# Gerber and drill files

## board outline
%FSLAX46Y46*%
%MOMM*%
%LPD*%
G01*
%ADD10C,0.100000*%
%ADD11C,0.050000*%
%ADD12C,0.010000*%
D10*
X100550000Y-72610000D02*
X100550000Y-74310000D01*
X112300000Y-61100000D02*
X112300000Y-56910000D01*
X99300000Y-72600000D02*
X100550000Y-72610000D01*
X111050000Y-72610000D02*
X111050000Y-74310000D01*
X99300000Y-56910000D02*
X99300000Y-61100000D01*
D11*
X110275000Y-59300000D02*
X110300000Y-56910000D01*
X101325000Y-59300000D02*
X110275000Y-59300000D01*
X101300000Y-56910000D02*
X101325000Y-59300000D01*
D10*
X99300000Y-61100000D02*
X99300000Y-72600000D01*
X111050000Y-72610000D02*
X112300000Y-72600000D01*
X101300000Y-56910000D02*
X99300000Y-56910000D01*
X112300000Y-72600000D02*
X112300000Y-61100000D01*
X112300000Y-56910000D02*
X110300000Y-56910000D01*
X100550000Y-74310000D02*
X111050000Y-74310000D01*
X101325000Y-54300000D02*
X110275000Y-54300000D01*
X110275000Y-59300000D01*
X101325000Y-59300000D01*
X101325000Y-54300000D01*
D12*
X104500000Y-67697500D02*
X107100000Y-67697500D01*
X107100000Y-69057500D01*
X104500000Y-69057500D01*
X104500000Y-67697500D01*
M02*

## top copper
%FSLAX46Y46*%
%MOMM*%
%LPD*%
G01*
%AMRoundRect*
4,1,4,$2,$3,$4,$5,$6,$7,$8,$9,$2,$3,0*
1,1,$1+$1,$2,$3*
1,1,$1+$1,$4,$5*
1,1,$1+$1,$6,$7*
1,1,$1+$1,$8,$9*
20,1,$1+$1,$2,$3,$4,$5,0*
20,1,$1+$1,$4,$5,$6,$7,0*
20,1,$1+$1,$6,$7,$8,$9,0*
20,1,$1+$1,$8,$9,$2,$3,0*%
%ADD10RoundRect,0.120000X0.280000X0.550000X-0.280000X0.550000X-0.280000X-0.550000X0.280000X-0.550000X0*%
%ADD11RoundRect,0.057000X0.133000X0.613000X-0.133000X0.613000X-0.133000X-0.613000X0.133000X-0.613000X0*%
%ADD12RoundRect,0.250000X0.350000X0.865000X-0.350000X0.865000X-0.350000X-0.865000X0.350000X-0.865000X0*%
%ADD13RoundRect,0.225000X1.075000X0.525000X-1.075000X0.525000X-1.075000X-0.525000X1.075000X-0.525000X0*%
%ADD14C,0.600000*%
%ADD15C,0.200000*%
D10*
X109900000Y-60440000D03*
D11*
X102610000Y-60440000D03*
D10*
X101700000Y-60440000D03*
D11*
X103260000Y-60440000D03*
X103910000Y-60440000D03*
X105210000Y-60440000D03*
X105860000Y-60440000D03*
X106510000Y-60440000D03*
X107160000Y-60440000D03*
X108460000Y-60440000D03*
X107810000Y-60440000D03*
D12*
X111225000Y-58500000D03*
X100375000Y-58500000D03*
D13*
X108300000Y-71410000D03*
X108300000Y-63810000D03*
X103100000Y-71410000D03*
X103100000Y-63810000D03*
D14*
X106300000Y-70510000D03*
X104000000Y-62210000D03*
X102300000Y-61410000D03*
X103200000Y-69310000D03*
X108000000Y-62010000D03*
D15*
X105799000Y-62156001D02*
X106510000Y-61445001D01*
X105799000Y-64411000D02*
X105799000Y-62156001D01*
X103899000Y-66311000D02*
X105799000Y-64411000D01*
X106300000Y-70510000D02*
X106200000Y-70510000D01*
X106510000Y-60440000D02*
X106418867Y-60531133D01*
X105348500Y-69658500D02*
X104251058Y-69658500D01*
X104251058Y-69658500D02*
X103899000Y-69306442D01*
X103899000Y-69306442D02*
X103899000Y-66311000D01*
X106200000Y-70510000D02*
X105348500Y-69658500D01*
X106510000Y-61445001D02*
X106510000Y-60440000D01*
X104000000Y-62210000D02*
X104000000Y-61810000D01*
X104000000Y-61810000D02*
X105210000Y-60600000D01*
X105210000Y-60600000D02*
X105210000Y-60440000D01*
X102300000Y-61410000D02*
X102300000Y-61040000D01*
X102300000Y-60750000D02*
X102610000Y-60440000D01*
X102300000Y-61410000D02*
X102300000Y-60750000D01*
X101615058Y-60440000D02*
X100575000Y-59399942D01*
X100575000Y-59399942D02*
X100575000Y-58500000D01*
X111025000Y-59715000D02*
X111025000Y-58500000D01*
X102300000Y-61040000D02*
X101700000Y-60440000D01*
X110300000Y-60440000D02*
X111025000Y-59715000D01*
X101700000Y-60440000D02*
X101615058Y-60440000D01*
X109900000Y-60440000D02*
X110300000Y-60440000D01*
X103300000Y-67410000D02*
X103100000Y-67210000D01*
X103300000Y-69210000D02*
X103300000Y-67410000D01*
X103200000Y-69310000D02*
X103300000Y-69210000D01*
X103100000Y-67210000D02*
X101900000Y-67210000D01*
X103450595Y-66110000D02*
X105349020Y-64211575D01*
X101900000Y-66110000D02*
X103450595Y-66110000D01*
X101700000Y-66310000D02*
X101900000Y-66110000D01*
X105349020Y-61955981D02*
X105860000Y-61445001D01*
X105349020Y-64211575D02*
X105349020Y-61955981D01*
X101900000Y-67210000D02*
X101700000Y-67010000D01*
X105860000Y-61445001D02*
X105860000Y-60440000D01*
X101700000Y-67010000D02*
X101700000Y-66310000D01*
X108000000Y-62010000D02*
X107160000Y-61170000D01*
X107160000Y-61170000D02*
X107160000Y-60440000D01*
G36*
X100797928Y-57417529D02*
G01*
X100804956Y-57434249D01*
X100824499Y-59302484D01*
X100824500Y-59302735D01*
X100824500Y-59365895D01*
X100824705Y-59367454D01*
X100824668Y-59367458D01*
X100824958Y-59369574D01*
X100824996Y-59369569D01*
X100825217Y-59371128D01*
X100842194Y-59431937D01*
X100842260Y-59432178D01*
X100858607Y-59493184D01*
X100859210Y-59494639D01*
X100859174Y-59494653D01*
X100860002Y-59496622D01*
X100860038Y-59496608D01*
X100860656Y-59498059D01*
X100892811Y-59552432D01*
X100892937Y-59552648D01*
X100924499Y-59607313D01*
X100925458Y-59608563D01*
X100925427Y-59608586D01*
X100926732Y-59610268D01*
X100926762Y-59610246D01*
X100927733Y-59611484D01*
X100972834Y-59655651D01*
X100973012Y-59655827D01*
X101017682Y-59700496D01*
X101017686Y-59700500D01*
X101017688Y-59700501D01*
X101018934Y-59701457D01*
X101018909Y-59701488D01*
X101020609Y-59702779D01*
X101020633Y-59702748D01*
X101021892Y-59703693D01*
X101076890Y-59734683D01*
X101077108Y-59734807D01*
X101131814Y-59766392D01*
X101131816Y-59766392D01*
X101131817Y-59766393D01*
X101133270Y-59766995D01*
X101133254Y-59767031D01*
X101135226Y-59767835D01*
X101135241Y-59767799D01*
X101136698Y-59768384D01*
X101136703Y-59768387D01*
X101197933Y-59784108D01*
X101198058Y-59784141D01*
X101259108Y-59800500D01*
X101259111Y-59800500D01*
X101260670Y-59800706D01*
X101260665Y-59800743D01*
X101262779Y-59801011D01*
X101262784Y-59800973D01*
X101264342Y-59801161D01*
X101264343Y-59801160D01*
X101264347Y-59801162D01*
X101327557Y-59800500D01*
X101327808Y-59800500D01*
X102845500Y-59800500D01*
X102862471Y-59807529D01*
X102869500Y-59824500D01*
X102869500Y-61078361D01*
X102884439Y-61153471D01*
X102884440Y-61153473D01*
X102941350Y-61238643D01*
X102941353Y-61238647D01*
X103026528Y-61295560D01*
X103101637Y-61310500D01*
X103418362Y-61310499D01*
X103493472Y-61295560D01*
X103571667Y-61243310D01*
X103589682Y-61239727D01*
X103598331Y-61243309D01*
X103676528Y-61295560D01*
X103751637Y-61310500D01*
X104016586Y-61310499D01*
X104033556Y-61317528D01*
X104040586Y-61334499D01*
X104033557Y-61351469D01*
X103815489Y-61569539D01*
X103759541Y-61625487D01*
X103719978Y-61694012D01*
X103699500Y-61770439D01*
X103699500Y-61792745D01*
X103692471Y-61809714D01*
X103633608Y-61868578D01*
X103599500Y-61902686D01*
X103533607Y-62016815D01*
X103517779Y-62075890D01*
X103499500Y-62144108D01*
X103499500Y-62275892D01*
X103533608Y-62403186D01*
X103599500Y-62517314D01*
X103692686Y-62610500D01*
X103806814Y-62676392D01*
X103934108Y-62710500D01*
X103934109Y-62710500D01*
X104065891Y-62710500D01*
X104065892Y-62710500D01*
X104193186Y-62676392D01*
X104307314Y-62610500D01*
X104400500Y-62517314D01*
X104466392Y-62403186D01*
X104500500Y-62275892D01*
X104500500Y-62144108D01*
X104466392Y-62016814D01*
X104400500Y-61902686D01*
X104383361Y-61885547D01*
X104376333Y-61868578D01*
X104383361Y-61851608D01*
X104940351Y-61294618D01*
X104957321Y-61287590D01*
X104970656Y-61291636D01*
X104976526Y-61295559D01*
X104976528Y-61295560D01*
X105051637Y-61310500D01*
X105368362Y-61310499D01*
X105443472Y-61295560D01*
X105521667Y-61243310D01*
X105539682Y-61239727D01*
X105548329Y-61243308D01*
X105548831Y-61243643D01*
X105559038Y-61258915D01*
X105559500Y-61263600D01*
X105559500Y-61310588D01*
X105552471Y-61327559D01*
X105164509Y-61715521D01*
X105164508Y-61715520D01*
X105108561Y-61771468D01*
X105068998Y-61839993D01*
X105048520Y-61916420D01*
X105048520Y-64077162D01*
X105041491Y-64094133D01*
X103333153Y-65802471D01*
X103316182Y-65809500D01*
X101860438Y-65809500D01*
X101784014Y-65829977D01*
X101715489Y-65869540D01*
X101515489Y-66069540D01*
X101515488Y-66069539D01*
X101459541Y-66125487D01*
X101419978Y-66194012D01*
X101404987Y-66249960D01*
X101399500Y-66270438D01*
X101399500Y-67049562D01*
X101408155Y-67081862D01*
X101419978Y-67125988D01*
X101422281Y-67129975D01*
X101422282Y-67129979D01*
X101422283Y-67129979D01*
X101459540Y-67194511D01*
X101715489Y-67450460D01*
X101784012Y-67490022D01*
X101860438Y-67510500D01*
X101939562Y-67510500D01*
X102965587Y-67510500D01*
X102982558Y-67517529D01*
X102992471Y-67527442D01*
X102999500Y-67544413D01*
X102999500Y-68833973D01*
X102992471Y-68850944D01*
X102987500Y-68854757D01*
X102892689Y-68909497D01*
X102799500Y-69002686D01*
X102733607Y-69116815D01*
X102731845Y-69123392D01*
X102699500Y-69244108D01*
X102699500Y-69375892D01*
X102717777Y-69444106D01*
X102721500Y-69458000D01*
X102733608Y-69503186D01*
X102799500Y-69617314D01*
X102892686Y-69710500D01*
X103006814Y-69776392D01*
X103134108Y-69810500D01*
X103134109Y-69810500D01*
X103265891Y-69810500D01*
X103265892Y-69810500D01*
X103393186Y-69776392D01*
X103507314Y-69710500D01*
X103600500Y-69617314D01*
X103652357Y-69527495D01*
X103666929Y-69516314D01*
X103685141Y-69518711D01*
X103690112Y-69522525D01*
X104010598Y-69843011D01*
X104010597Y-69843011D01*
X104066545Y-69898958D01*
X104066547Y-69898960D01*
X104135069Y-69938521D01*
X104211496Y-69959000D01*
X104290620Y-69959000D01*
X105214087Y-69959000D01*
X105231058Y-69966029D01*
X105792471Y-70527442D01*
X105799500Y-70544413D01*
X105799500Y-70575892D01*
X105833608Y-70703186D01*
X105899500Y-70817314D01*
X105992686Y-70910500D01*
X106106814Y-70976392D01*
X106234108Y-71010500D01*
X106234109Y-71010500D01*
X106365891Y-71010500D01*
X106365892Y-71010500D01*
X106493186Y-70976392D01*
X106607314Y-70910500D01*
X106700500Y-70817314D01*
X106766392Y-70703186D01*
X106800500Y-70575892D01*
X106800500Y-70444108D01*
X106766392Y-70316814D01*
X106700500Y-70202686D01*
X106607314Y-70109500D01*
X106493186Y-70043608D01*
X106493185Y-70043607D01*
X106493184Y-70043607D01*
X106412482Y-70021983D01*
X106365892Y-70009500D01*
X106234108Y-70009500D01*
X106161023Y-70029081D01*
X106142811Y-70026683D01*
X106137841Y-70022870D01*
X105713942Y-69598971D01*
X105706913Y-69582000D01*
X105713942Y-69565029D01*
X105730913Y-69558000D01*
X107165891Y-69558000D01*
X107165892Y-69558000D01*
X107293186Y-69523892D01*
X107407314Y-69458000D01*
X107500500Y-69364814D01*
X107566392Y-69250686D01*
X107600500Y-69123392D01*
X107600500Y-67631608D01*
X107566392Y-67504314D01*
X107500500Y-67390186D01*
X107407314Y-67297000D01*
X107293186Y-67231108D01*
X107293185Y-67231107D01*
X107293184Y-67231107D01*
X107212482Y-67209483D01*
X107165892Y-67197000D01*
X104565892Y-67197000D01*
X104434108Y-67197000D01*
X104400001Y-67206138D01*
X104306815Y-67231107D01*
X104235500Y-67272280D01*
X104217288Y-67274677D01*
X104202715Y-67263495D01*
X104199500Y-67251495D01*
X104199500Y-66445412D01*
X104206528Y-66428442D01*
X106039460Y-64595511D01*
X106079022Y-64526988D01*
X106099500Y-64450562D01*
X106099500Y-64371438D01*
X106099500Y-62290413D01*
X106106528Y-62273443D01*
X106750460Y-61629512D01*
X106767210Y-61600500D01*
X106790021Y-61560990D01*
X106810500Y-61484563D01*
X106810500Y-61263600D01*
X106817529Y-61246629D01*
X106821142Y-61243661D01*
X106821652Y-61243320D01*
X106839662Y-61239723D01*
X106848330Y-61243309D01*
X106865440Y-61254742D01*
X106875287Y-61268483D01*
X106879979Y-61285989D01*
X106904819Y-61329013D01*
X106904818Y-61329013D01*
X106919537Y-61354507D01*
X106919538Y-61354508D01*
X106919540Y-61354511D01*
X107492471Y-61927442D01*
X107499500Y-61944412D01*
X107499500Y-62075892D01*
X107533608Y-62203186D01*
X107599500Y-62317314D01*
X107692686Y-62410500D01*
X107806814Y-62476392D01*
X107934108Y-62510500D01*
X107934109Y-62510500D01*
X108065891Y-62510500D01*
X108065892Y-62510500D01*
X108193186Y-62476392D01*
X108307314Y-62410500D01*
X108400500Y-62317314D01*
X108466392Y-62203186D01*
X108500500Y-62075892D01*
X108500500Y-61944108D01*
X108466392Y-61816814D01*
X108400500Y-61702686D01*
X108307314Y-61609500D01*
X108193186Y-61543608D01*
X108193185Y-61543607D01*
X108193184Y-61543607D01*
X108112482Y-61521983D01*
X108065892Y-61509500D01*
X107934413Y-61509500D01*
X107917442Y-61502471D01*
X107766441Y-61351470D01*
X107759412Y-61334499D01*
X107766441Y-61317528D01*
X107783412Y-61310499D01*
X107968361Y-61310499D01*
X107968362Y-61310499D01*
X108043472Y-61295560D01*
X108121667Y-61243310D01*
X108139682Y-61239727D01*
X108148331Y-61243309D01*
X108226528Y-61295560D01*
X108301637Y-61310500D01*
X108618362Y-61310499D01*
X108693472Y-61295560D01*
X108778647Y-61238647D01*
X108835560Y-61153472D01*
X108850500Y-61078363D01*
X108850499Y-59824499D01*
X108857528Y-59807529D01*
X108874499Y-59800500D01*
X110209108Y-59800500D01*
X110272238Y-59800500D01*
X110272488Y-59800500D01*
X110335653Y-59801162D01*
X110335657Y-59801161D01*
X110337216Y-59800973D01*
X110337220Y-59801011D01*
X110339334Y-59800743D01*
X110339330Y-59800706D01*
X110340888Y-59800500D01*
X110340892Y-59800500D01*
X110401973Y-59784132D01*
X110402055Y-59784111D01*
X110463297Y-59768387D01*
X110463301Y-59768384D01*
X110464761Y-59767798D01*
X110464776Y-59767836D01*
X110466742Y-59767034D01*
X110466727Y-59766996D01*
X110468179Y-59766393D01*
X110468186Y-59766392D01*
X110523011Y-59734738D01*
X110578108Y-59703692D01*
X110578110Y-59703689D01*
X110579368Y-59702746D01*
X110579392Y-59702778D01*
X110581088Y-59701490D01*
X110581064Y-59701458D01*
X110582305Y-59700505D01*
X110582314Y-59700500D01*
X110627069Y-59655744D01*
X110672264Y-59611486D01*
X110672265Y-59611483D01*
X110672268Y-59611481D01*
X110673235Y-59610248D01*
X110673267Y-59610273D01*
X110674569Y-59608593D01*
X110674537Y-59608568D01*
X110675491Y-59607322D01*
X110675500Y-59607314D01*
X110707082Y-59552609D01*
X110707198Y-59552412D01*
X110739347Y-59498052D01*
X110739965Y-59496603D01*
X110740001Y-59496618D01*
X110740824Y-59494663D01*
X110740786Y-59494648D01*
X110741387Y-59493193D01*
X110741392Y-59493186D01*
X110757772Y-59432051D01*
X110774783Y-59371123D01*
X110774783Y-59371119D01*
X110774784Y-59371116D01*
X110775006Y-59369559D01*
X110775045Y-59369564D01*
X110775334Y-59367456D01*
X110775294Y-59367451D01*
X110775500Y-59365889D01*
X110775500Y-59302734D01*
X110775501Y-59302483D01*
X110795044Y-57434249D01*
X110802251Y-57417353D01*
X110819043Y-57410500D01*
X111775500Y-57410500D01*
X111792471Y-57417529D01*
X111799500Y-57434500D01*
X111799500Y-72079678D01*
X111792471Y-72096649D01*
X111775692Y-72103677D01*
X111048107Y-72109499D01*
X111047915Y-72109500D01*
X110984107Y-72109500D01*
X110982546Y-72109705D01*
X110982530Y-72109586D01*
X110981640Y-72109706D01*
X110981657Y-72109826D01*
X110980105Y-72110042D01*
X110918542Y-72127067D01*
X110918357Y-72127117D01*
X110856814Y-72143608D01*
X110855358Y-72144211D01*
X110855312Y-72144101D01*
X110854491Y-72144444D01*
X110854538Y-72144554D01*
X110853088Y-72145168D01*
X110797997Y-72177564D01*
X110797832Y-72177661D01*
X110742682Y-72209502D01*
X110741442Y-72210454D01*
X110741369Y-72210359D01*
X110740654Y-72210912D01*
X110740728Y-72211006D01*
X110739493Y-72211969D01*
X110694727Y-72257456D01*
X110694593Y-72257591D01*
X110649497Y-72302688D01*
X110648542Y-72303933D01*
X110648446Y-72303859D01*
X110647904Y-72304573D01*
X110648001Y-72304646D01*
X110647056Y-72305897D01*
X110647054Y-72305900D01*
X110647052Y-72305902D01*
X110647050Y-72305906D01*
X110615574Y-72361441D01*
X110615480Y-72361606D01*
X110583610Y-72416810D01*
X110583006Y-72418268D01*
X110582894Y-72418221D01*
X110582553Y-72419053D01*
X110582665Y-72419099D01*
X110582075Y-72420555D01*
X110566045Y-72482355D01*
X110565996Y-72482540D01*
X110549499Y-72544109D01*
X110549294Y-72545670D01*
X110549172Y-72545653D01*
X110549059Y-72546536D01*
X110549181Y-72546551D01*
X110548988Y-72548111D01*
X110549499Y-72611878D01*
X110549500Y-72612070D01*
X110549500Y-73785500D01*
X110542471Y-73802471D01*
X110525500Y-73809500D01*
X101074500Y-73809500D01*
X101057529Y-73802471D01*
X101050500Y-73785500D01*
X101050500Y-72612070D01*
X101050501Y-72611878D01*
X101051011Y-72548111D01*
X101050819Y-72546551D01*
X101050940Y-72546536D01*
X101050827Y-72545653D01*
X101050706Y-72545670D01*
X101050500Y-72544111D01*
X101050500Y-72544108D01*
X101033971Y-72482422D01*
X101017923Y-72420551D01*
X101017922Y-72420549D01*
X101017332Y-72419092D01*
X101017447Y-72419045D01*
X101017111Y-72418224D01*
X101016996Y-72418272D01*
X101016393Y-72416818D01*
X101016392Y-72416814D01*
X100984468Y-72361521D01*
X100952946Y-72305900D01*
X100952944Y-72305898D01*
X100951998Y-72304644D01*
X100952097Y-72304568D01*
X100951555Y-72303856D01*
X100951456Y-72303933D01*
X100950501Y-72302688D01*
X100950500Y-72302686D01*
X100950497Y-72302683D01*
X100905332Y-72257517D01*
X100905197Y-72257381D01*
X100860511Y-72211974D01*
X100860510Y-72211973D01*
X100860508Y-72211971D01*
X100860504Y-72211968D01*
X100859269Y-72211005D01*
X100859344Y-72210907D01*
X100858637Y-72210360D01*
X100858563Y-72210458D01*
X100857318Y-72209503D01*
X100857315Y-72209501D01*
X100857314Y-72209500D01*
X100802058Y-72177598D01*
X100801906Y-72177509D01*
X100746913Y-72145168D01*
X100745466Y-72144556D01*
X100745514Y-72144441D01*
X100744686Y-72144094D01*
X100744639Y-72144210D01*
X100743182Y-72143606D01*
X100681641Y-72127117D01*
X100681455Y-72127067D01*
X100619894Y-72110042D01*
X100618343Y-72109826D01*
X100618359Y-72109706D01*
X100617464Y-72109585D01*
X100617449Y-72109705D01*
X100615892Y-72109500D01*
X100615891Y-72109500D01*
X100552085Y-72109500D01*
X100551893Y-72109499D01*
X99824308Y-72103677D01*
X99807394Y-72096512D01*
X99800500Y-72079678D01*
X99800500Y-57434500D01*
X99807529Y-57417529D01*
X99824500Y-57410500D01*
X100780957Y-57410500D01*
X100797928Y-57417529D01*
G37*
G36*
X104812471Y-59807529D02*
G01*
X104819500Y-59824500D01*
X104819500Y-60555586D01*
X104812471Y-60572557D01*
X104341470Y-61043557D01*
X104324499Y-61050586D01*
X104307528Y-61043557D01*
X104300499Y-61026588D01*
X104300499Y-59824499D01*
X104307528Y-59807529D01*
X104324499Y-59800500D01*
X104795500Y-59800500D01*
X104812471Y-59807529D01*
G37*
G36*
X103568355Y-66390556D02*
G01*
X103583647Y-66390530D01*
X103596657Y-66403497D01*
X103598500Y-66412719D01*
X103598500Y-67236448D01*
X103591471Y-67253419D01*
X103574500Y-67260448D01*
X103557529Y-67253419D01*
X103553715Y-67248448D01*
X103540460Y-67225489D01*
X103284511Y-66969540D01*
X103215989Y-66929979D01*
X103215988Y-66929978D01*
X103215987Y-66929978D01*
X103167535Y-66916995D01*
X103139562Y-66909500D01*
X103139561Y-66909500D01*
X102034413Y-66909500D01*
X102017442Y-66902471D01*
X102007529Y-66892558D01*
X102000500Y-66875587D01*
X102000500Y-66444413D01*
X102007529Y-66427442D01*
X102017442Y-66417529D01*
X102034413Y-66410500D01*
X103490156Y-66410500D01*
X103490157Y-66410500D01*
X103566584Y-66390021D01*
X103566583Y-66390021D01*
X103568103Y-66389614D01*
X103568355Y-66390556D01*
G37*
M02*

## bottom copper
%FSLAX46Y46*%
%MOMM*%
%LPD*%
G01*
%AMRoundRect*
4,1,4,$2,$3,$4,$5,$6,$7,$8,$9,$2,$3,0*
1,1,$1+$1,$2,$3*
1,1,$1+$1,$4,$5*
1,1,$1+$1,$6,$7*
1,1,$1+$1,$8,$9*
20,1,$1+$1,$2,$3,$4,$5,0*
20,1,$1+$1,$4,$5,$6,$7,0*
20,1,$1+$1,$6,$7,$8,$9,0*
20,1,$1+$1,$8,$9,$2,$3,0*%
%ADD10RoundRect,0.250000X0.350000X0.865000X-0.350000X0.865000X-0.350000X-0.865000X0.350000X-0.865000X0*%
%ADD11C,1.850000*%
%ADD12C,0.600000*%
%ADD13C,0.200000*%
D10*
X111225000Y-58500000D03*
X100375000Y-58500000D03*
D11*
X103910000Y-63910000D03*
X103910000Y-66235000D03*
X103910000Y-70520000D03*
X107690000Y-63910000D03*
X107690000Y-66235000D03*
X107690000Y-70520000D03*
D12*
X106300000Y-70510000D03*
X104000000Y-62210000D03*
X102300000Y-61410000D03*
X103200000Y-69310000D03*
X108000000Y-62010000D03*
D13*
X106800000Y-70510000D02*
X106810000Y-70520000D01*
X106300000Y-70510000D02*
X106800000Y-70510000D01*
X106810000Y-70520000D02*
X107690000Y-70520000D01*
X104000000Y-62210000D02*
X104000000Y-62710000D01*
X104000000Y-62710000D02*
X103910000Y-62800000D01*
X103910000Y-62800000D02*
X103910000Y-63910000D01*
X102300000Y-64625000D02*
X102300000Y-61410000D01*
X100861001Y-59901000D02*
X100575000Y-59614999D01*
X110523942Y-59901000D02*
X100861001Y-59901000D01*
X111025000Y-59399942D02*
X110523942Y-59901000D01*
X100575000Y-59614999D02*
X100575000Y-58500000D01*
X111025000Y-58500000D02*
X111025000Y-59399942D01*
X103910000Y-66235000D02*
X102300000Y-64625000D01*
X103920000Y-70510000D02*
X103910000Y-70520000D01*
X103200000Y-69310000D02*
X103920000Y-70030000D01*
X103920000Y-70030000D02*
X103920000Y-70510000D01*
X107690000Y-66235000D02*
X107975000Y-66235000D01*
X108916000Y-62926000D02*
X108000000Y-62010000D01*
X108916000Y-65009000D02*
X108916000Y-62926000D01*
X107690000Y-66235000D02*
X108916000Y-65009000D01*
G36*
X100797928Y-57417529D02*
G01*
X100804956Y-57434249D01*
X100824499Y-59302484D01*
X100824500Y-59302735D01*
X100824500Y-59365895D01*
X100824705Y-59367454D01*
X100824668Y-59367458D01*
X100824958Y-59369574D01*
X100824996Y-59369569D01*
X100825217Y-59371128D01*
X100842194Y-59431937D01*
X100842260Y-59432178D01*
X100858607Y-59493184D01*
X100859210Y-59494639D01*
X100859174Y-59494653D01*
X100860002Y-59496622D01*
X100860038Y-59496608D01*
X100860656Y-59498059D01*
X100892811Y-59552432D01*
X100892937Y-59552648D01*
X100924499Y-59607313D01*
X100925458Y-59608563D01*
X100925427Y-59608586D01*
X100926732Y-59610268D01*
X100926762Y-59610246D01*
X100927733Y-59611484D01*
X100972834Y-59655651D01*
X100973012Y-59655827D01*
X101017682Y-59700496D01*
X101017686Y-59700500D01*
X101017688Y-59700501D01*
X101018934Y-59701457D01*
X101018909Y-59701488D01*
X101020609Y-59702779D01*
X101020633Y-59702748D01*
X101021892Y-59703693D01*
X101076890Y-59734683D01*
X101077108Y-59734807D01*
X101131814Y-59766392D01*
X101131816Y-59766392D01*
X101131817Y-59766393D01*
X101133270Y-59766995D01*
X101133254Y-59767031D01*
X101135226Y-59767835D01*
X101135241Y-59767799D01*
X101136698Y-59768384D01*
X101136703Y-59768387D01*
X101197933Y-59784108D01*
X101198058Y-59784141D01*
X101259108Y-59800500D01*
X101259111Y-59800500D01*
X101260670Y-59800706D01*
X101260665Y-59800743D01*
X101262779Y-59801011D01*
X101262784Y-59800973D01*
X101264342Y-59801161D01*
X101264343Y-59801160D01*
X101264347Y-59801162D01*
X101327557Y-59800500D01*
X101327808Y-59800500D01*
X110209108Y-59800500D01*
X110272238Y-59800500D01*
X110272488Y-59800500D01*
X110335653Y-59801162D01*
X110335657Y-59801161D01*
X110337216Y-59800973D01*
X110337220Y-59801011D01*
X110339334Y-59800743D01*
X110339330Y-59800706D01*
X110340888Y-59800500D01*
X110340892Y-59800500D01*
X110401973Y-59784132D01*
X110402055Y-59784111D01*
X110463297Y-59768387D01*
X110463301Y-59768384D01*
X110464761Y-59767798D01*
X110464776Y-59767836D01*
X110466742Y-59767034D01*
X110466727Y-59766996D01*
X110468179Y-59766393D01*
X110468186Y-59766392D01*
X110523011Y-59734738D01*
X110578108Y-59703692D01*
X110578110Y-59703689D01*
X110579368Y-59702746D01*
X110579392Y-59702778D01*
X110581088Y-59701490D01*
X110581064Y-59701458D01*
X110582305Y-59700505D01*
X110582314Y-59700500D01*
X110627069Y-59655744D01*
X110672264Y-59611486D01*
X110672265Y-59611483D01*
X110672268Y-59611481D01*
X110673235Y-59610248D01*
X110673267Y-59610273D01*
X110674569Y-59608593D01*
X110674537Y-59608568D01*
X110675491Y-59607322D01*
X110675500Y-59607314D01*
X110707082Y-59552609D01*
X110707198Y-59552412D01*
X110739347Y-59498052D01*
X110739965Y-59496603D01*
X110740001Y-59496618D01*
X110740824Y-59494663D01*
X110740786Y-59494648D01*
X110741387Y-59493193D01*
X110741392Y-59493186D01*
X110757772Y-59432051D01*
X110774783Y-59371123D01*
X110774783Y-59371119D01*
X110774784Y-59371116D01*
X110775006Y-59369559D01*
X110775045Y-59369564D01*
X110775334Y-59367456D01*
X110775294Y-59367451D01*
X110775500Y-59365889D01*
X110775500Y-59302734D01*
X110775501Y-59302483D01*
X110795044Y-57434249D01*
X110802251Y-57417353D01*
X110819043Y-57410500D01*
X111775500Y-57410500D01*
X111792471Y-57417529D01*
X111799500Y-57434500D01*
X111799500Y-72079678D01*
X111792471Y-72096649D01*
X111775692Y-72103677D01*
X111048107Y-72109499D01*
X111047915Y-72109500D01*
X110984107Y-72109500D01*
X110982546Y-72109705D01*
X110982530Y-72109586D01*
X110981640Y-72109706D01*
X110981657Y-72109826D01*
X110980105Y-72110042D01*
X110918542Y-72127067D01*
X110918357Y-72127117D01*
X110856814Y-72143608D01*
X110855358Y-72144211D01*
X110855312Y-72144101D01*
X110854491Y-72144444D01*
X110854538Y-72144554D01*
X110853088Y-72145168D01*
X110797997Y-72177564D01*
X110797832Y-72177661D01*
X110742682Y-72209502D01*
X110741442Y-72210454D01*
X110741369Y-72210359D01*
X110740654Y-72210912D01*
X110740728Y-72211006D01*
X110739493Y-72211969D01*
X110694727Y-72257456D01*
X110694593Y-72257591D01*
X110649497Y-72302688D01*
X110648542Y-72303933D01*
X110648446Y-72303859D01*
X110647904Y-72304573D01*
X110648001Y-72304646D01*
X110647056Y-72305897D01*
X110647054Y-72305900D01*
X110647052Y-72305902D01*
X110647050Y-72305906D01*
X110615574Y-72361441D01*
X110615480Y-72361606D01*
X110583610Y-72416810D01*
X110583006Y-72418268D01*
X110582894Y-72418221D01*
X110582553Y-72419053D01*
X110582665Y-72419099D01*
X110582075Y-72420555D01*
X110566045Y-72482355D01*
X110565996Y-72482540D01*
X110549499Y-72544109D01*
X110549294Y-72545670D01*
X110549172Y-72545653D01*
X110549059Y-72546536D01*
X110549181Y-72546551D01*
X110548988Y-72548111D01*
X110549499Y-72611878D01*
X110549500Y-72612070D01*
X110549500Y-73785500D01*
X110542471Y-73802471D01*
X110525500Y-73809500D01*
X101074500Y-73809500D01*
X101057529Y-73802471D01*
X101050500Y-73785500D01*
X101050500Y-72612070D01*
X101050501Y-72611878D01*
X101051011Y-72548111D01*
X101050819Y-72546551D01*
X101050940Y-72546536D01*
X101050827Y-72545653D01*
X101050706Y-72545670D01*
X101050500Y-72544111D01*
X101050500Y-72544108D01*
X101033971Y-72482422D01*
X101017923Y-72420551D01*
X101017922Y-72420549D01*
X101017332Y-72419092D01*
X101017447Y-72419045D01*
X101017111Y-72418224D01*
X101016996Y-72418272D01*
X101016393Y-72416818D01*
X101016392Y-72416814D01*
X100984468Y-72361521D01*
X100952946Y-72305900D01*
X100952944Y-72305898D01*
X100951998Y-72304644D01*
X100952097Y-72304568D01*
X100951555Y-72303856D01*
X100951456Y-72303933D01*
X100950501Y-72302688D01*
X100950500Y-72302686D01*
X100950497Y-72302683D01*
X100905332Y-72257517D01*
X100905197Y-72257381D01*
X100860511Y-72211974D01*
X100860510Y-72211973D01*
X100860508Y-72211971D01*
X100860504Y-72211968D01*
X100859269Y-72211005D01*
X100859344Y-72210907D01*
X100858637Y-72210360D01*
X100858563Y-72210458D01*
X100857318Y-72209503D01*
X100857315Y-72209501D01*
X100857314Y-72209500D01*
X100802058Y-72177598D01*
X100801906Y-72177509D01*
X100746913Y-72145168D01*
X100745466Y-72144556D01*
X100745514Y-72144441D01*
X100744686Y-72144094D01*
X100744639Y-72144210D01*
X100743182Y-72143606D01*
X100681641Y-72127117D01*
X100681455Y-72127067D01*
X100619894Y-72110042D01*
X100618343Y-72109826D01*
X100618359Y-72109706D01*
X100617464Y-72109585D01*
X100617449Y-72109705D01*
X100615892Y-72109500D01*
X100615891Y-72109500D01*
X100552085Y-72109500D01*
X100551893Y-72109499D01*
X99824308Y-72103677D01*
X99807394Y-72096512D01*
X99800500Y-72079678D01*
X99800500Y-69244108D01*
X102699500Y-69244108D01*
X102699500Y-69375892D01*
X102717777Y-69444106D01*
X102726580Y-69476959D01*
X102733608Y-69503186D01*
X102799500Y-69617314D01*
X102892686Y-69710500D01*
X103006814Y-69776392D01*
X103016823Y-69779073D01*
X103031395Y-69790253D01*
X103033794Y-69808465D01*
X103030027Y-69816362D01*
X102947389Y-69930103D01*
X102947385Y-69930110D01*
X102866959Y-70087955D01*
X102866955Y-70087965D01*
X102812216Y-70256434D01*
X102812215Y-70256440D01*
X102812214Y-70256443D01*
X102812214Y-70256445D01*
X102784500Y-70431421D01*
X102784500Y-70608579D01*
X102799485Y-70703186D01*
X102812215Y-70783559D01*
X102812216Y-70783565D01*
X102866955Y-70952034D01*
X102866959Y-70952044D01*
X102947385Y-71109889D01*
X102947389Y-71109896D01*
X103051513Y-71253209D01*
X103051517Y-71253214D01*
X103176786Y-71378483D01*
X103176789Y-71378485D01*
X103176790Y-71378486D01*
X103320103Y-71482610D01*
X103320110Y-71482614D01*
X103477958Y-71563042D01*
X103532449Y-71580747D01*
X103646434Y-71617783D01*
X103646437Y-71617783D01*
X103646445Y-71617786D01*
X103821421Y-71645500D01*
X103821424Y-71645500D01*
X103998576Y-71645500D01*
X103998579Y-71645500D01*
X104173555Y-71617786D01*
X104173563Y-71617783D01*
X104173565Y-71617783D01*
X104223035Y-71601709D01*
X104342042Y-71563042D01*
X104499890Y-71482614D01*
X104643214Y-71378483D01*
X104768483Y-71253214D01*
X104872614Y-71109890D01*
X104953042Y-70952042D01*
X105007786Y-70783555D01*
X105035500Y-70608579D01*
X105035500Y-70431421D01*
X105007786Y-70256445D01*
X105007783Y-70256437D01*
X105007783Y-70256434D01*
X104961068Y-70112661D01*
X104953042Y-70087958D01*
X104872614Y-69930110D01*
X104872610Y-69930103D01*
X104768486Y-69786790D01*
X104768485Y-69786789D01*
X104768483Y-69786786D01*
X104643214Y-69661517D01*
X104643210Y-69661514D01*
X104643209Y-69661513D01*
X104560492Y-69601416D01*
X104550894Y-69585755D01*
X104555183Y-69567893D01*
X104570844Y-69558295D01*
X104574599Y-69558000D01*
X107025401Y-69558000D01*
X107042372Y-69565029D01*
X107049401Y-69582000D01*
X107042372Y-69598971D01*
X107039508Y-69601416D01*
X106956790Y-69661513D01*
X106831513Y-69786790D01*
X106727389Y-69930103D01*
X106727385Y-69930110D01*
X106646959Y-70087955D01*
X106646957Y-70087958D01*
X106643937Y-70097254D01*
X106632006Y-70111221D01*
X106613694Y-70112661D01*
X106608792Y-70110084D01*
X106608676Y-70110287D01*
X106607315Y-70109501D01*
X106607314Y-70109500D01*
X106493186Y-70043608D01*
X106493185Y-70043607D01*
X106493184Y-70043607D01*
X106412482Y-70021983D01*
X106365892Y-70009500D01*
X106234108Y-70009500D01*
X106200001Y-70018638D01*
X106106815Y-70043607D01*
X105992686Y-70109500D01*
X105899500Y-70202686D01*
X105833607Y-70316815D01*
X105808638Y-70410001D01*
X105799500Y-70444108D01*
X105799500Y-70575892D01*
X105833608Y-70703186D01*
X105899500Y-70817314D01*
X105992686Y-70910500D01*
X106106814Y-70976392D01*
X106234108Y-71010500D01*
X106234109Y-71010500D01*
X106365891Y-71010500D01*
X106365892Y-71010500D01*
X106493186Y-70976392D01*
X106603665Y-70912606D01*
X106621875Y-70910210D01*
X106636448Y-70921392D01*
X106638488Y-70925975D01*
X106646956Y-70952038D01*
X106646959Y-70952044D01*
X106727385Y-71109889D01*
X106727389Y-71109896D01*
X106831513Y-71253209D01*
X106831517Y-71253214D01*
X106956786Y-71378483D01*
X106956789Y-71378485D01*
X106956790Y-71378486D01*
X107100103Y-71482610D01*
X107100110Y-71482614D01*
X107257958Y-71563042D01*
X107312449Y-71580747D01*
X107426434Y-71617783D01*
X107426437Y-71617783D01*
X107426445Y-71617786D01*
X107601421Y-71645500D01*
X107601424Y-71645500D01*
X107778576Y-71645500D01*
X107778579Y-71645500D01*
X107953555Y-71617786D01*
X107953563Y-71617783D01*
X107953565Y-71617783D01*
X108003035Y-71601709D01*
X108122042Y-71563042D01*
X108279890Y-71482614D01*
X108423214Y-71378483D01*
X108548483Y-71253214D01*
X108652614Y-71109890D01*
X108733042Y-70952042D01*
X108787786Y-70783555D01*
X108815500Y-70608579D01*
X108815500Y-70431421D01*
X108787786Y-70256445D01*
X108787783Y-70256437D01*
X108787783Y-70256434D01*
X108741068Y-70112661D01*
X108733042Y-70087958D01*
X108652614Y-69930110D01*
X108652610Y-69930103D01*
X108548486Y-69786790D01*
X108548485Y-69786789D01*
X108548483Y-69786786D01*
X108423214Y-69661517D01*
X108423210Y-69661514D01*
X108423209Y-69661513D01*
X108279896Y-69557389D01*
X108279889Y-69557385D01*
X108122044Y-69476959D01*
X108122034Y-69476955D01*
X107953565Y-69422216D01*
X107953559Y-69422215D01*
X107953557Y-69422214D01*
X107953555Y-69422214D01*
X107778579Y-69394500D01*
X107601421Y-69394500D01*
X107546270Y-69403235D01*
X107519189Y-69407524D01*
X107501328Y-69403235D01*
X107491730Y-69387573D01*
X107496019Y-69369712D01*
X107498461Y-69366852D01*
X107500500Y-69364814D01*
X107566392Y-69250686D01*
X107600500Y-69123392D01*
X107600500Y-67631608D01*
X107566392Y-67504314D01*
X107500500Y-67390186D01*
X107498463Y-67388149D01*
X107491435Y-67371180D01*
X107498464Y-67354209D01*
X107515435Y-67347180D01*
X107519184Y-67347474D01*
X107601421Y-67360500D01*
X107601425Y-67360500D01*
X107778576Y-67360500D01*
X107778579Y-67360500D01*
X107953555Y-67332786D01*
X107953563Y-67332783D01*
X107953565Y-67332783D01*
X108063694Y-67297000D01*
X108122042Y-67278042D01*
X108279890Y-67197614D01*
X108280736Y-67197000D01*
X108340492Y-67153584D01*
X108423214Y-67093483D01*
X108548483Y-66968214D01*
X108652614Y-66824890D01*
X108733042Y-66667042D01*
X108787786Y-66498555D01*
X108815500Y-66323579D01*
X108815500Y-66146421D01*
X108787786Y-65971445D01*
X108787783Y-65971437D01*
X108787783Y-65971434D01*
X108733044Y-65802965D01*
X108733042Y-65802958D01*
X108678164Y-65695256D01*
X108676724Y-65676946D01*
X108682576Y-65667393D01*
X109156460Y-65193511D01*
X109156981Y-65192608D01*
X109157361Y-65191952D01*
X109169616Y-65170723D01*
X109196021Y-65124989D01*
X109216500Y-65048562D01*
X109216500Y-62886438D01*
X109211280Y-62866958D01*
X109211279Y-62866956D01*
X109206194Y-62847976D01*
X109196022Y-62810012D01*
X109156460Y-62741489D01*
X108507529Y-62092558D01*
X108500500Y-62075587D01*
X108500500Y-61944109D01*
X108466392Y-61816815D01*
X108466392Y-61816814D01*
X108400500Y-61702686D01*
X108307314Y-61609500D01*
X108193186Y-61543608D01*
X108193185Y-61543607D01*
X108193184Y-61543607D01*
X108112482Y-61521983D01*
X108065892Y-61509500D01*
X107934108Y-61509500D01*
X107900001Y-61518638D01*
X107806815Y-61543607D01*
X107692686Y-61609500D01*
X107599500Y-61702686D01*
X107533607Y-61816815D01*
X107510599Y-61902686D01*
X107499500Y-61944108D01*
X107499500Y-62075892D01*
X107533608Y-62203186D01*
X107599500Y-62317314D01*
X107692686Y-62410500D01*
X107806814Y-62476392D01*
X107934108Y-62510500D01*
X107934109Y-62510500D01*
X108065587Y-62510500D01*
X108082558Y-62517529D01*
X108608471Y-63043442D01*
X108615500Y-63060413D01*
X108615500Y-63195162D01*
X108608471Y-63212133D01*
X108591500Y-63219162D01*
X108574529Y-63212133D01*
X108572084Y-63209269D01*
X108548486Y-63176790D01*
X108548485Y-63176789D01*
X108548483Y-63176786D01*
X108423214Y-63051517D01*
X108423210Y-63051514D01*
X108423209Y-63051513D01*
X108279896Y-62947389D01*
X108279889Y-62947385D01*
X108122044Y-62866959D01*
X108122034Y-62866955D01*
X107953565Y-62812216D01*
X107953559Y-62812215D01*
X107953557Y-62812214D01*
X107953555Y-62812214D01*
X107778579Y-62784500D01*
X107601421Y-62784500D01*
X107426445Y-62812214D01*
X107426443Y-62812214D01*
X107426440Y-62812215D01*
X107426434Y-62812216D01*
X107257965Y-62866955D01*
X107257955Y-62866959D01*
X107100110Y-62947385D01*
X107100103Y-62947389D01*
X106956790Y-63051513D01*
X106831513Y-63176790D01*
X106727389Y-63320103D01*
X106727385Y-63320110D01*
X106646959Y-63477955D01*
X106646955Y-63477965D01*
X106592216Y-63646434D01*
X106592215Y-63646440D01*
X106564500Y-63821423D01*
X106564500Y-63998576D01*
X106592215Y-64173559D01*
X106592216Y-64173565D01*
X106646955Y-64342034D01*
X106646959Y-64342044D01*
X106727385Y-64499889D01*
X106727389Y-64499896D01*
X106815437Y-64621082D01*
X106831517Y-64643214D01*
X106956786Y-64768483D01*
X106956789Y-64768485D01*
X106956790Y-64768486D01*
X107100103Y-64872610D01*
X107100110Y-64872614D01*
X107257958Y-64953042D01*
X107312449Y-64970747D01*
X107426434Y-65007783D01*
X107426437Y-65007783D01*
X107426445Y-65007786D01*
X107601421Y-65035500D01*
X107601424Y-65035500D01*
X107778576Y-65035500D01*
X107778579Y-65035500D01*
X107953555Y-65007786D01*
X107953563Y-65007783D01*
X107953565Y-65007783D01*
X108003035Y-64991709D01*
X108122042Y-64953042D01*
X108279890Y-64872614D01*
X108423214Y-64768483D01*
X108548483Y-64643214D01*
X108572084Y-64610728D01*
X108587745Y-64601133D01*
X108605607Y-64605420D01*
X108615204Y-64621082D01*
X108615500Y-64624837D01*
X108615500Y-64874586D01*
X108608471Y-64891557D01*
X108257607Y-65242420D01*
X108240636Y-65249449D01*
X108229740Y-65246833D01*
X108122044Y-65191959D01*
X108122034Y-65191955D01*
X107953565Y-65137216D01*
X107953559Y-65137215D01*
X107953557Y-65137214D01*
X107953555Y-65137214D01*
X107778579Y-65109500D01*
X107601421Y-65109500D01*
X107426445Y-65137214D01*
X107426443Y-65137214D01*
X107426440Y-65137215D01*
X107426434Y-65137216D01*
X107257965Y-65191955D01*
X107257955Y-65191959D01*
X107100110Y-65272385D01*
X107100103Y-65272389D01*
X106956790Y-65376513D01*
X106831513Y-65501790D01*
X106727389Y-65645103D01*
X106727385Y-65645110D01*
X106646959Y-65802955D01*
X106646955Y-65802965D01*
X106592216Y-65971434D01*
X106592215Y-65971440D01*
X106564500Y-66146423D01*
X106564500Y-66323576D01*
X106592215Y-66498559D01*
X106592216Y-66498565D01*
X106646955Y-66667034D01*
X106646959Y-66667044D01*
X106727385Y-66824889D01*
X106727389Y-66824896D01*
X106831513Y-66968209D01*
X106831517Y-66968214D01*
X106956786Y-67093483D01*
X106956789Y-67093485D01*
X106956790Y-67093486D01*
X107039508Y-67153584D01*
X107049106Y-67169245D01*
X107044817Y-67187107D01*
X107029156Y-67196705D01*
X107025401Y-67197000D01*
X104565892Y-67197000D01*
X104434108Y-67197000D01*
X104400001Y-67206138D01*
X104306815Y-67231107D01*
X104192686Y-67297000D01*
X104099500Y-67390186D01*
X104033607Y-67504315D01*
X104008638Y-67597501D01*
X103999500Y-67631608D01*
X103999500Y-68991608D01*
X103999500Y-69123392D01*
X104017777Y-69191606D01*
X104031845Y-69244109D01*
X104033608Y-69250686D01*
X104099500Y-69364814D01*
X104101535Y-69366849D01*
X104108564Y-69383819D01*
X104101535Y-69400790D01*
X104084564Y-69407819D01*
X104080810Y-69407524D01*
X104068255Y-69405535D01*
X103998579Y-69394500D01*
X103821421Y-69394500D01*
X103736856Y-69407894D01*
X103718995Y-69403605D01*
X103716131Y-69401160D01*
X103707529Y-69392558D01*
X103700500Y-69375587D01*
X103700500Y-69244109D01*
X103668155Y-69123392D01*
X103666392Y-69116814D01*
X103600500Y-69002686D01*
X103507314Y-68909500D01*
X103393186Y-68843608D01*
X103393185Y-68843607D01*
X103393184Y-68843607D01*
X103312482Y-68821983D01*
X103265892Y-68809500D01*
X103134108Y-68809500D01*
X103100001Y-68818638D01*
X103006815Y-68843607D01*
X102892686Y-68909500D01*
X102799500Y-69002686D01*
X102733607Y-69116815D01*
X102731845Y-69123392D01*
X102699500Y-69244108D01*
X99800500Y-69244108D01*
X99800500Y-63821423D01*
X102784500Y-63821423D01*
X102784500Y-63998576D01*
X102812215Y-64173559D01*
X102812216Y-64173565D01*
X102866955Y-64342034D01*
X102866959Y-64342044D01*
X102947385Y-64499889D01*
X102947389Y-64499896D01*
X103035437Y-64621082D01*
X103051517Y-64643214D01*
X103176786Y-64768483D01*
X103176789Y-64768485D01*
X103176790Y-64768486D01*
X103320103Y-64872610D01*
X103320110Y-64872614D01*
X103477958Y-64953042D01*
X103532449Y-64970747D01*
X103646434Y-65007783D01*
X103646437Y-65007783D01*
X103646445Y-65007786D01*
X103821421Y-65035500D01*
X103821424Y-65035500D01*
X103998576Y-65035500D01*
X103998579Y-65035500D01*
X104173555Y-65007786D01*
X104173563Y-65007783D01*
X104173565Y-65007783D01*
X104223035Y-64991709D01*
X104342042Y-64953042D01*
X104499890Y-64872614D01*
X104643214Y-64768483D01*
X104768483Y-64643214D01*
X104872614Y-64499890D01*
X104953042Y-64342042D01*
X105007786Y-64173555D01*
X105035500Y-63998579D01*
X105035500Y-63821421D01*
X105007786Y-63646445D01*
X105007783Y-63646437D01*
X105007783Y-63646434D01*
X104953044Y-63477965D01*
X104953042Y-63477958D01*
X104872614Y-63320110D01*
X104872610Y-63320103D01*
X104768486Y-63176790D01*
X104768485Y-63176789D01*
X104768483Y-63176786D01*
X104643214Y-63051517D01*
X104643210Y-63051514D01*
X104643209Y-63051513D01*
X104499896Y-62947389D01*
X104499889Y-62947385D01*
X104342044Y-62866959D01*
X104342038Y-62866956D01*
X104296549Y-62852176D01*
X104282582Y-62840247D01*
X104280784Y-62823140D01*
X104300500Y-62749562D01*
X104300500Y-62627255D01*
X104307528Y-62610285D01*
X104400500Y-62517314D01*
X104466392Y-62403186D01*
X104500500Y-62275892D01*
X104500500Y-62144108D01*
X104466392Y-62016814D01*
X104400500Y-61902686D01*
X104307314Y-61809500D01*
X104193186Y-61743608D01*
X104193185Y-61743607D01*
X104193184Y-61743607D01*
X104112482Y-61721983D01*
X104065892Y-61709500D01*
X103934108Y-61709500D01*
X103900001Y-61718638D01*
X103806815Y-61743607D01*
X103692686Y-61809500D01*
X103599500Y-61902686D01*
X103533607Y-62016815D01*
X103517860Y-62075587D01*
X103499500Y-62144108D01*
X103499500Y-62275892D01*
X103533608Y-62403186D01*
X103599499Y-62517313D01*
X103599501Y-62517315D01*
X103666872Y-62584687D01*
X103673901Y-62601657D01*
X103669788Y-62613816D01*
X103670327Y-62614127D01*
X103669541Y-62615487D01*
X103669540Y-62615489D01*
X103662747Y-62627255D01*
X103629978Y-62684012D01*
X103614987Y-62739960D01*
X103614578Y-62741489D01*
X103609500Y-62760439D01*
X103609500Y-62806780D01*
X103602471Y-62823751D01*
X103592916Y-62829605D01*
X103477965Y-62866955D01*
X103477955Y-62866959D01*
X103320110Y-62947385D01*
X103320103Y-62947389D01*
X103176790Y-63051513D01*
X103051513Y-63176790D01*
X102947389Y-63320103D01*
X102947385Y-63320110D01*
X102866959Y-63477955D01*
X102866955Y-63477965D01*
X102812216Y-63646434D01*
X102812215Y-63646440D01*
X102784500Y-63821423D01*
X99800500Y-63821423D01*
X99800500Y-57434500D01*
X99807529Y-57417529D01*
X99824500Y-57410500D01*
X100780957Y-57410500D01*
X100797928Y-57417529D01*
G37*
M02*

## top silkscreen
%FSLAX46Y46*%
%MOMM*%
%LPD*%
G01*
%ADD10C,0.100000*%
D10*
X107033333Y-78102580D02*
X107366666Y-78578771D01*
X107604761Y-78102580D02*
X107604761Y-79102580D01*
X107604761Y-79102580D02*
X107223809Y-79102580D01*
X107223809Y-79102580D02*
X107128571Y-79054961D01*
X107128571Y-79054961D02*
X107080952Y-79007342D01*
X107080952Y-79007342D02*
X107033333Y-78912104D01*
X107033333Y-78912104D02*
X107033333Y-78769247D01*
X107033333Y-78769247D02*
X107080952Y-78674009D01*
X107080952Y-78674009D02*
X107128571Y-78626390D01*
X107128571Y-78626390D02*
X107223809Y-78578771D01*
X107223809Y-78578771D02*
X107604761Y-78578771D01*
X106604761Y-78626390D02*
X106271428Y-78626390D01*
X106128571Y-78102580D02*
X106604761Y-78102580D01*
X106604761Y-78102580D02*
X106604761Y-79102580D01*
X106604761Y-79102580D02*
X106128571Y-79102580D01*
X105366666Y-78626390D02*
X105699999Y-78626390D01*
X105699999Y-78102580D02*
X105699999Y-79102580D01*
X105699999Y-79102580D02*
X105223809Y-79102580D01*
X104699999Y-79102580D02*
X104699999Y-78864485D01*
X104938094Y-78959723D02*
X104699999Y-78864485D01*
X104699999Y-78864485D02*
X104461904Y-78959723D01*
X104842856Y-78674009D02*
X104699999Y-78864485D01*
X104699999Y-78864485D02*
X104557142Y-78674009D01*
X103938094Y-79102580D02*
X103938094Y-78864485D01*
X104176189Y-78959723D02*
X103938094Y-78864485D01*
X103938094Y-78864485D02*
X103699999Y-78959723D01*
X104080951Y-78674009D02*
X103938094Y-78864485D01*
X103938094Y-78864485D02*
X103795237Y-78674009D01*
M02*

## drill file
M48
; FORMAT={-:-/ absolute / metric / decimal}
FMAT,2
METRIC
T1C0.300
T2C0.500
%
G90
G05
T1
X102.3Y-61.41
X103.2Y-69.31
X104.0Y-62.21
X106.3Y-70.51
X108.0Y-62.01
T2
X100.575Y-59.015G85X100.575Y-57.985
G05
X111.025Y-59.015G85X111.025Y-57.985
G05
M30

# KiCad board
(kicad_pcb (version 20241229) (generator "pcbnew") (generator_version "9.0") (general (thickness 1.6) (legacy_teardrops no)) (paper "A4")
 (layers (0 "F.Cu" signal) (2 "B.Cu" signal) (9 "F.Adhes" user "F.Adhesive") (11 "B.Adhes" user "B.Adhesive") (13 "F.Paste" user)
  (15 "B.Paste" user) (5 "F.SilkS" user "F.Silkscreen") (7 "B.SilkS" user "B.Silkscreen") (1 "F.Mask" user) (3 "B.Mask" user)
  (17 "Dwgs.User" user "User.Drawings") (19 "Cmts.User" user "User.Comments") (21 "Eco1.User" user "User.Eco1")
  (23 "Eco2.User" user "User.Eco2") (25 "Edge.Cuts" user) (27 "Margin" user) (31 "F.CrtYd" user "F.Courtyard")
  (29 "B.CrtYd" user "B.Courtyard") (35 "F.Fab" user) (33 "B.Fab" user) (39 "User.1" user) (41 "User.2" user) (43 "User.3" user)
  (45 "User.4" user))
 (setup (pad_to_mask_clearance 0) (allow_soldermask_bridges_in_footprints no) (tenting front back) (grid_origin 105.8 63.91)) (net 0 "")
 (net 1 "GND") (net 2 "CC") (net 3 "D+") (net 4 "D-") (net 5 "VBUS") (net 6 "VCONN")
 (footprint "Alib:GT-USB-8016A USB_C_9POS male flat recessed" (layer "F.Cu") (at 105.8 62 180)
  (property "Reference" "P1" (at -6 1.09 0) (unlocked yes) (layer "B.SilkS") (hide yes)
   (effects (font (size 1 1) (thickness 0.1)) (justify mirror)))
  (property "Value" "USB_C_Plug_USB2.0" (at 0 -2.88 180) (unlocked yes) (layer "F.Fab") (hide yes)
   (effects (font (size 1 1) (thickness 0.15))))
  (fp_rect (start -4.475 2.7) (end 4.475 7.7) (stroke (width 0.1) (type solid)) (fill no) (layer "Edge.Cuts"))
  (pad "A1" smd roundrect (at -4.1 1.56 180) (size 0.8 1.34) (layers "F.Cu" "F.Mask" "F.Paste") (roundrect_rratio 0.15) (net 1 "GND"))
  (pad "A1" smd roundrect (at 3.19 1.56 180) (size 0.38 1.34) (layers "F.Cu" "F.Mask" "F.Paste") (roundrect_rratio 0.15) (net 1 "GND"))
  (pad "A1" smd roundrect (at 4.1 1.56 180) (size 0.8 1.34) (layers "F.Cu" "F.Mask" "F.Paste") (roundrect_rratio 0.15) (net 1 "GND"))
  (pad "A2" smd roundrect (at 2.54 1.56 180) (size 0.38 1.34) (layers "F.Cu" "F.Mask" "F.Paste") (roundrect_rratio 0.15))
  (pad "A3" smd roundrect (at 1.89 1.56 180) (size 0.38 1.34) (layers "F.Cu" "F.Mask" "F.Paste") (roundrect_rratio 0.15))
  (pad "A5" smd roundrect (at 0.59 1.56 180) (size 0.38 1.34) (layers "F.Cu" "F.Mask" "F.Paste") (roundrect_rratio 0.15) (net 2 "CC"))
  (pad "A6" smd roundrect (at -0.06 1.56 180) (size 0.38 1.34) (layers "F.Cu" "F.Mask" "F.Paste") (roundrect_rratio 0.15) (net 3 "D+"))
  (pad "A7" smd roundrect (at -0.71 1.56 180) (size 0.38 1.34) (layers "F.Cu" "F.Mask" "F.Paste") (roundrect_rratio 0.15) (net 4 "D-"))
  (pad "A9" smd roundrect (at -1.36 1.56 180) (size 0.38 1.34) (layers "F.Cu" "F.Mask" "F.Paste") (roundrect_rratio 0.15) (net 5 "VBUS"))
  (pad "B10" smd roundrect (at -2.66 1.56 180) (size 0.38 1.34) (layers "F.Cu" "F.Mask" "F.Paste") (roundrect_rratio 0.15))
  (pad "B11" smd roundrect (at -2.01 1.56 180) (size 0.38 1.34) (layers "F.Cu" "F.Mask" "F.Paste") (roundrect_rratio 0.15))
  (pad "S1" thru_hole roundrect (at -5.225 3.5 180) (size 1.2 2.23) (drill oval 0.5 1.53 (offset -0.2 0)) (layers "*.Cu" "*.Mask")
   (remove_unused_layers no) (roundrect_rratio 0.2083333333) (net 1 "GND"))
  (pad "S1" thru_hole roundrect (at 5.225 3.5 180) (size 1.2 2.23) (drill oval 0.5 1.53 (offset 0.2 0)) (layers "*.Cu" "*.Mask")
   (remove_unused_layers no) (roundrect_rratio 0.2083333333) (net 1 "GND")))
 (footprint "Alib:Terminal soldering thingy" (layer "F.Cu") (at 105.7 78.06 180)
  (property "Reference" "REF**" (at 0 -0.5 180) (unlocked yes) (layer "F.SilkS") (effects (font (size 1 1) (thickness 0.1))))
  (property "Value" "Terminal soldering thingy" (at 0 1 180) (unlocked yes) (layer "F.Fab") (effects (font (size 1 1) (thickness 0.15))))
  (pad "1" smd roundrect (at -2.6 6.65 180) (size 2.6 1.5) (layers "F.Cu" "F.Mask" "F.Paste") (roundrect_rratio 0.15) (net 1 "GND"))
  (pad "1" smd roundrect (at -2.6 14.25 180) (size 2.6 1.5) (layers "F.Cu" "F.Mask" "F.Paste") (roundrect_rratio 0.15) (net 1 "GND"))
  (pad "1" smd roundrect (at 2.6 6.65 180) (size 2.6 1.5) (layers "F.Cu" "F.Mask" "F.Paste") (roundrect_rratio 0.15) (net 1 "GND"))
  (pad "1" smd roundrect (at 2.6 14.25 180) (size 2.6 1.5) (layers "F.Cu" "F.Mask" "F.Paste") (roundrect_rratio 0.15) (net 1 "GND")))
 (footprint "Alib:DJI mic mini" (layer "B.Cu") (at 105.8 63.91 180)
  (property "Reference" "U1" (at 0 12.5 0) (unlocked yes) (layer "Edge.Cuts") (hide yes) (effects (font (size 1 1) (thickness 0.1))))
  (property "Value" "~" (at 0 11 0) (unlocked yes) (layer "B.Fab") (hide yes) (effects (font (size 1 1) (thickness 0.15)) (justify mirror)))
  (fp_rect (start -1.3 -3.7875) (end 1.3 -5.1475) (stroke (width 0.01) (type solid)) (fill no) (layer "Edge.Cuts"))
  (pad "1" smd circle (at 1.89 0 180) (size 1.85 1.85) (layers "B.Cu" "B.Mask" "B.Paste") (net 2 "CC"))
  (pad "2" smd circle (at 1.89 -2.325 180) (size 1.85 1.85) (layers "B.Cu" "B.Mask" "B.Paste") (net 1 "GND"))
  (pad "3" smd circle (at 1.89 -6.61 180) (size 1.85 1.85) (layers "B.Cu" "B.Mask" "B.Paste") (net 3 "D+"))
  (pad "4" smd circle (at -1.89 0 180) (size 1.85 1.85) (layers "B.Cu" "B.Mask" "B.Paste") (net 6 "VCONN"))
  (pad "5" smd circle (at -1.89 -2.325 180) (size 1.85 1.85) (layers "B.Cu" "B.Mask" "B.Paste") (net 5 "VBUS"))
  (pad "6" smd circle (at -1.89 -6.61 180) (size 1.85 1.85) (layers "B.Cu" "B.Mask" "B.Paste") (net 4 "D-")))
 (gr_line (start 100.55 72.61) (end 100.55 74.31) (stroke (width 0.1) (type solid)) (layer "Edge.Cuts"))
 (gr_line (start 112.3 61.1) (end 112.3 56.91) (stroke (width 0.1) (type solid)) (layer "Edge.Cuts"))
 (gr_line (start 99.3 72.6) (end 100.55 72.61) (stroke (width 0.1) (type solid)) (layer "Edge.Cuts"))
 (gr_line (start 111.05 72.61) (end 111.05 74.31) (stroke (width 0.1) (type solid)) (layer "Edge.Cuts"))
 (gr_line (start 99.3 56.91) (end 99.3 61.1) (stroke (width 0.1) (type solid)) (layer "Edge.Cuts"))
 (gr_line (start 110.275 59.3) (end 110.3 56.91) (stroke (width 0.05) (type solid)) (layer "Edge.Cuts"))
 (gr_line (start 101.325 59.3) (end 110.275 59.3) (stroke (width 0.05) (type default)) (layer "Edge.Cuts"))
 (gr_line (start 101.3 56.91) (end 101.325 59.3) (stroke (width 0.05) (type default)) (layer "Edge.Cuts"))
 (gr_line (start 99.3 61.1) (end 99.3 72.6) (stroke (width 0.1) (type solid)) (layer "Edge.Cuts"))
 (gr_line (start 111.05 72.61) (end 112.3 72.6) (stroke (width 0.1) (type solid)) (layer "Edge.Cuts"))
 (gr_line (start 101.3 56.91) (end 99.3 56.91) (stroke (width 0.1) (type solid)) (layer "Edge.Cuts"))
 (gr_line (start 112.3 72.6) (end 112.3 61.1) (stroke (width 0.1) (type solid)) (layer "Edge.Cuts"))
 (gr_line (start 112.3 56.91) (end 110.3 56.91) (stroke (width 0.1) (type solid)) (layer "Edge.Cuts"))
 (gr_line (start 100.55 74.31) (end 111.05 74.31) (stroke (width 0.1) (type solid)) (layer "Edge.Cuts"))
 (segment (start 105.799 62.156001) (end 106.51 61.445001) (width 0.2) (layer "F.Cu") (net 4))
 (segment (start 105.799 64.411) (end 105.799 62.156001) (width 0.2) (layer "F.Cu") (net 4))
 (segment (start 103.899 66.311) (end 105.799 64.411) (width 0.2) (layer "F.Cu") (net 4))
 (segment (start 106.3 70.51) (end 106.2 70.51) (width 0.2) (layer "F.Cu") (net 4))
 (segment (start 106.51 60.44) (end 106.418867 60.531133) (width 0.2) (layer "F.Cu") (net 4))
 (segment (start 105.3485 69.6585) (end 104.251058 69.6585) (width 0.2) (layer "F.Cu") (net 4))
 (segment (start 104.251058 69.6585) (end 103.899 69.306442) (width 0.2) (layer "F.Cu") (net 4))
 (segment (start 103.899 69.306442) (end 103.899 66.311) (width 0.2) (layer "F.Cu") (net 4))
 (segment (start 106.2 70.51) (end 105.3485 69.6585) (width 0.2) (layer "F.Cu") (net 4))
 (segment (start 106.51 61.445001) (end 106.51 60.44) (width 0.2) (layer "F.Cu") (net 4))
 (via (at 106.3 70.51) (size 0.6) (drill 0.3) (layers "F.Cu" "B.Cu") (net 4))
 (segment (start 106.8 70.51) (end 106.81 70.52) (width 0.2) (layer "B.Cu") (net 4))
 (segment (start 106.3 70.51) (end 106.8 70.51) (width 0.2) (layer "B.Cu") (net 4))
 (segment (start 106.81 70.52) (end 107.69 70.52) (width 0.2) (layer "B.Cu") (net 4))
 (segment (start 104 62.21) (end 104 61.81) (width 0.2) (layer "F.Cu") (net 2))
 (segment (start 104 61.81) (end 105.21 60.6) (width 0.2) (layer "F.Cu") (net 2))
 (segment (start 105.21 60.6) (end 105.21 60.44) (width 0.2) (layer "F.Cu") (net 2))
 (via (at 104 62.21) (size 0.6) (drill 0.3) (layers "F.Cu" "B.Cu") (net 2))
 (segment (start 104 62.21) (end 104 62.71) (width 0.2) (layer "B.Cu") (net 2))
 (segment (start 104 62.71) (end 103.91 62.8) (width 0.2) (layer "B.Cu") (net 2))
 (segment (start 103.91 62.8) (end 103.91 63.91) (width 0.2) (layer "B.Cu") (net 2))
 (segment (start 102.3 61.41) (end 102.3 61.04) (width 0.2) (layer "F.Cu") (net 1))
 (segment (start 102.3 60.75) (end 102.61 60.44) (width 0.2) (layer "F.Cu") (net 1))
 (segment (start 102.3 61.41) (end 102.3 60.75) (width 0.2) (layer "F.Cu") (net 1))
 (segment (start 101.615058 60.44) (end 100.575 59.399942) (width 0.2) (layer "F.Cu") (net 1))
 (segment (start 100.575 59.399942) (end 100.575 58.5) (width 0.2) (layer "F.Cu") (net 1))
 (segment (start 111.025 59.715) (end 111.025 58.5) (width 0.2) (layer "F.Cu") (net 1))
 (segment (start 102.3 61.04) (end 101.7 60.44) (width 0.2) (layer "F.Cu") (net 1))
 (segment (start 110.3 60.44) (end 111.025 59.715) (width 0.2) (layer "F.Cu") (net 1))
 (segment (start 101.7 60.44) (end 101.615058 60.44) (width 0.2) (layer "F.Cu") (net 1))
 (segment (start 109.9 60.44) (end 110.3 60.44) (width 0.2) (layer "F.Cu") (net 1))
 (via (at 102.3 61.41) (size 0.6) (drill 0.3) (layers "F.Cu" "B.Cu") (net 1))
 (segment (start 102.3 64.625) (end 102.3 61.41) (width 0.2) (layer "B.Cu") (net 1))
 (segment (start 100.861001 59.901) (end 100.575 59.614999) (width 0.2) (layer "B.Cu") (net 1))
 (segment (start 110.523942 59.901) (end 100.861001 59.901) (width 0.2) (layer "B.Cu") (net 1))
 (segment (start 111.025 59.399942) (end 110.523942 59.901) (width 0.2) (layer "B.Cu") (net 1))
 (segment (start 100.575 59.614999) (end 100.575 58.5) (width 0.2) (layer "B.Cu") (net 1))
 (segment (start 111.025 58.5) (end 111.025 59.399942) (width 0.2) (layer "B.Cu") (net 1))
 (segment (start 103.91 66.235) (end 102.3 64.625) (width 0.2) (layer "B.Cu") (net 1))
 (segment (start 103.3 67.41) (end 103.1 67.21) (width 0.2) (layer "F.Cu") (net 3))
 (segment (start 103.3 69.21) (end 103.3 67.41) (width 0.2) (layer "F.Cu") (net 3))
 (segment (start 103.2 69.31) (end 103.3 69.21) (width 0.2) (layer "F.Cu") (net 3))
 (segment (start 103.1 67.21) (end 101.9 67.21) (width 0.2) (layer "F.Cu") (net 3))
 (segment (start 103.450595 66.11) (end 105.34902 64.211575) (width 0.2) (layer "F.Cu") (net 3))
 (segment (start 101.9 66.11) (end 103.450595 66.11) (width 0.2) (layer "F.Cu") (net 3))
 (segment (start 101.7 66.31) (end 101.9 66.11) (width 0.2) (layer "F.Cu") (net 3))
 (segment (start 105.34902 61.955981) (end 105.86 61.445001) (width 0.2) (layer "F.Cu") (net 3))
 (segment (start 105.34902 64.211575) (end 105.34902 61.955981) (width 0.2) (layer "F.Cu") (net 3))
 (segment (start 101.9 67.21) (end 101.7 67.01) (width 0.2) (layer "F.Cu") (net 3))
 (segment (start 105.86 61.445001) (end 105.86 60.44) (width 0.2) (layer "F.Cu") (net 3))
 (segment (start 101.7 67.01) (end 101.7 66.31) (width 0.2) (layer "F.Cu") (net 3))
 (via (at 103.2 69.31) (size 0.6) (drill 0.3) (layers "F.Cu" "B.Cu") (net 3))
 (segment (start 103.92 70.51) (end 103.91 70.52) (width 0.2) (layer "B.Cu") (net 3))
 (segment (start 103.2 69.31) (end 103.92 70.03) (width 0.2) (layer "B.Cu") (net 3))
 (segment (start 103.92 70.03) (end 103.92 70.51) (width 0.2) (layer "B.Cu") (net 3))
 (segment (start 108 62.01) (end 107.16 61.17) (width 0.2) (layer "F.Cu") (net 5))
 (segment (start 107.16 61.17) (end 107.16 60.44) (width 0.2) (layer "F.Cu") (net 5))
 (via (at 108 62.01) (size 0.6) (drill 0.3) (layers "F.Cu" "B.Cu") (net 5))
 (segment (start 107.69 66.235) (end 107.975 66.235) (width 0.2) (layer "B.Cu") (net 5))
 (segment (start 108.916 62.926) (end 108 62.01) (width 0.2) (layer "B.Cu") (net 5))
 (segment (start 108.916 65.009) (end 108.916 62.926) (width 0.2) (layer "B.Cu") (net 5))
 (segment (start 107.69 66.235) (end 108.916 65.009) (width 0.2) (layer "B.Cu") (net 5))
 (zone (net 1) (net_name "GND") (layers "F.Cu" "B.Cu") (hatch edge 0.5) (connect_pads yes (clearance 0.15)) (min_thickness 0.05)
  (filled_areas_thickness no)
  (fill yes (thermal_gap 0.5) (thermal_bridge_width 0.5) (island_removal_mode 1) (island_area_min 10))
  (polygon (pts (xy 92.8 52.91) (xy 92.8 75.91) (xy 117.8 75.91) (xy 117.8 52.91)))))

